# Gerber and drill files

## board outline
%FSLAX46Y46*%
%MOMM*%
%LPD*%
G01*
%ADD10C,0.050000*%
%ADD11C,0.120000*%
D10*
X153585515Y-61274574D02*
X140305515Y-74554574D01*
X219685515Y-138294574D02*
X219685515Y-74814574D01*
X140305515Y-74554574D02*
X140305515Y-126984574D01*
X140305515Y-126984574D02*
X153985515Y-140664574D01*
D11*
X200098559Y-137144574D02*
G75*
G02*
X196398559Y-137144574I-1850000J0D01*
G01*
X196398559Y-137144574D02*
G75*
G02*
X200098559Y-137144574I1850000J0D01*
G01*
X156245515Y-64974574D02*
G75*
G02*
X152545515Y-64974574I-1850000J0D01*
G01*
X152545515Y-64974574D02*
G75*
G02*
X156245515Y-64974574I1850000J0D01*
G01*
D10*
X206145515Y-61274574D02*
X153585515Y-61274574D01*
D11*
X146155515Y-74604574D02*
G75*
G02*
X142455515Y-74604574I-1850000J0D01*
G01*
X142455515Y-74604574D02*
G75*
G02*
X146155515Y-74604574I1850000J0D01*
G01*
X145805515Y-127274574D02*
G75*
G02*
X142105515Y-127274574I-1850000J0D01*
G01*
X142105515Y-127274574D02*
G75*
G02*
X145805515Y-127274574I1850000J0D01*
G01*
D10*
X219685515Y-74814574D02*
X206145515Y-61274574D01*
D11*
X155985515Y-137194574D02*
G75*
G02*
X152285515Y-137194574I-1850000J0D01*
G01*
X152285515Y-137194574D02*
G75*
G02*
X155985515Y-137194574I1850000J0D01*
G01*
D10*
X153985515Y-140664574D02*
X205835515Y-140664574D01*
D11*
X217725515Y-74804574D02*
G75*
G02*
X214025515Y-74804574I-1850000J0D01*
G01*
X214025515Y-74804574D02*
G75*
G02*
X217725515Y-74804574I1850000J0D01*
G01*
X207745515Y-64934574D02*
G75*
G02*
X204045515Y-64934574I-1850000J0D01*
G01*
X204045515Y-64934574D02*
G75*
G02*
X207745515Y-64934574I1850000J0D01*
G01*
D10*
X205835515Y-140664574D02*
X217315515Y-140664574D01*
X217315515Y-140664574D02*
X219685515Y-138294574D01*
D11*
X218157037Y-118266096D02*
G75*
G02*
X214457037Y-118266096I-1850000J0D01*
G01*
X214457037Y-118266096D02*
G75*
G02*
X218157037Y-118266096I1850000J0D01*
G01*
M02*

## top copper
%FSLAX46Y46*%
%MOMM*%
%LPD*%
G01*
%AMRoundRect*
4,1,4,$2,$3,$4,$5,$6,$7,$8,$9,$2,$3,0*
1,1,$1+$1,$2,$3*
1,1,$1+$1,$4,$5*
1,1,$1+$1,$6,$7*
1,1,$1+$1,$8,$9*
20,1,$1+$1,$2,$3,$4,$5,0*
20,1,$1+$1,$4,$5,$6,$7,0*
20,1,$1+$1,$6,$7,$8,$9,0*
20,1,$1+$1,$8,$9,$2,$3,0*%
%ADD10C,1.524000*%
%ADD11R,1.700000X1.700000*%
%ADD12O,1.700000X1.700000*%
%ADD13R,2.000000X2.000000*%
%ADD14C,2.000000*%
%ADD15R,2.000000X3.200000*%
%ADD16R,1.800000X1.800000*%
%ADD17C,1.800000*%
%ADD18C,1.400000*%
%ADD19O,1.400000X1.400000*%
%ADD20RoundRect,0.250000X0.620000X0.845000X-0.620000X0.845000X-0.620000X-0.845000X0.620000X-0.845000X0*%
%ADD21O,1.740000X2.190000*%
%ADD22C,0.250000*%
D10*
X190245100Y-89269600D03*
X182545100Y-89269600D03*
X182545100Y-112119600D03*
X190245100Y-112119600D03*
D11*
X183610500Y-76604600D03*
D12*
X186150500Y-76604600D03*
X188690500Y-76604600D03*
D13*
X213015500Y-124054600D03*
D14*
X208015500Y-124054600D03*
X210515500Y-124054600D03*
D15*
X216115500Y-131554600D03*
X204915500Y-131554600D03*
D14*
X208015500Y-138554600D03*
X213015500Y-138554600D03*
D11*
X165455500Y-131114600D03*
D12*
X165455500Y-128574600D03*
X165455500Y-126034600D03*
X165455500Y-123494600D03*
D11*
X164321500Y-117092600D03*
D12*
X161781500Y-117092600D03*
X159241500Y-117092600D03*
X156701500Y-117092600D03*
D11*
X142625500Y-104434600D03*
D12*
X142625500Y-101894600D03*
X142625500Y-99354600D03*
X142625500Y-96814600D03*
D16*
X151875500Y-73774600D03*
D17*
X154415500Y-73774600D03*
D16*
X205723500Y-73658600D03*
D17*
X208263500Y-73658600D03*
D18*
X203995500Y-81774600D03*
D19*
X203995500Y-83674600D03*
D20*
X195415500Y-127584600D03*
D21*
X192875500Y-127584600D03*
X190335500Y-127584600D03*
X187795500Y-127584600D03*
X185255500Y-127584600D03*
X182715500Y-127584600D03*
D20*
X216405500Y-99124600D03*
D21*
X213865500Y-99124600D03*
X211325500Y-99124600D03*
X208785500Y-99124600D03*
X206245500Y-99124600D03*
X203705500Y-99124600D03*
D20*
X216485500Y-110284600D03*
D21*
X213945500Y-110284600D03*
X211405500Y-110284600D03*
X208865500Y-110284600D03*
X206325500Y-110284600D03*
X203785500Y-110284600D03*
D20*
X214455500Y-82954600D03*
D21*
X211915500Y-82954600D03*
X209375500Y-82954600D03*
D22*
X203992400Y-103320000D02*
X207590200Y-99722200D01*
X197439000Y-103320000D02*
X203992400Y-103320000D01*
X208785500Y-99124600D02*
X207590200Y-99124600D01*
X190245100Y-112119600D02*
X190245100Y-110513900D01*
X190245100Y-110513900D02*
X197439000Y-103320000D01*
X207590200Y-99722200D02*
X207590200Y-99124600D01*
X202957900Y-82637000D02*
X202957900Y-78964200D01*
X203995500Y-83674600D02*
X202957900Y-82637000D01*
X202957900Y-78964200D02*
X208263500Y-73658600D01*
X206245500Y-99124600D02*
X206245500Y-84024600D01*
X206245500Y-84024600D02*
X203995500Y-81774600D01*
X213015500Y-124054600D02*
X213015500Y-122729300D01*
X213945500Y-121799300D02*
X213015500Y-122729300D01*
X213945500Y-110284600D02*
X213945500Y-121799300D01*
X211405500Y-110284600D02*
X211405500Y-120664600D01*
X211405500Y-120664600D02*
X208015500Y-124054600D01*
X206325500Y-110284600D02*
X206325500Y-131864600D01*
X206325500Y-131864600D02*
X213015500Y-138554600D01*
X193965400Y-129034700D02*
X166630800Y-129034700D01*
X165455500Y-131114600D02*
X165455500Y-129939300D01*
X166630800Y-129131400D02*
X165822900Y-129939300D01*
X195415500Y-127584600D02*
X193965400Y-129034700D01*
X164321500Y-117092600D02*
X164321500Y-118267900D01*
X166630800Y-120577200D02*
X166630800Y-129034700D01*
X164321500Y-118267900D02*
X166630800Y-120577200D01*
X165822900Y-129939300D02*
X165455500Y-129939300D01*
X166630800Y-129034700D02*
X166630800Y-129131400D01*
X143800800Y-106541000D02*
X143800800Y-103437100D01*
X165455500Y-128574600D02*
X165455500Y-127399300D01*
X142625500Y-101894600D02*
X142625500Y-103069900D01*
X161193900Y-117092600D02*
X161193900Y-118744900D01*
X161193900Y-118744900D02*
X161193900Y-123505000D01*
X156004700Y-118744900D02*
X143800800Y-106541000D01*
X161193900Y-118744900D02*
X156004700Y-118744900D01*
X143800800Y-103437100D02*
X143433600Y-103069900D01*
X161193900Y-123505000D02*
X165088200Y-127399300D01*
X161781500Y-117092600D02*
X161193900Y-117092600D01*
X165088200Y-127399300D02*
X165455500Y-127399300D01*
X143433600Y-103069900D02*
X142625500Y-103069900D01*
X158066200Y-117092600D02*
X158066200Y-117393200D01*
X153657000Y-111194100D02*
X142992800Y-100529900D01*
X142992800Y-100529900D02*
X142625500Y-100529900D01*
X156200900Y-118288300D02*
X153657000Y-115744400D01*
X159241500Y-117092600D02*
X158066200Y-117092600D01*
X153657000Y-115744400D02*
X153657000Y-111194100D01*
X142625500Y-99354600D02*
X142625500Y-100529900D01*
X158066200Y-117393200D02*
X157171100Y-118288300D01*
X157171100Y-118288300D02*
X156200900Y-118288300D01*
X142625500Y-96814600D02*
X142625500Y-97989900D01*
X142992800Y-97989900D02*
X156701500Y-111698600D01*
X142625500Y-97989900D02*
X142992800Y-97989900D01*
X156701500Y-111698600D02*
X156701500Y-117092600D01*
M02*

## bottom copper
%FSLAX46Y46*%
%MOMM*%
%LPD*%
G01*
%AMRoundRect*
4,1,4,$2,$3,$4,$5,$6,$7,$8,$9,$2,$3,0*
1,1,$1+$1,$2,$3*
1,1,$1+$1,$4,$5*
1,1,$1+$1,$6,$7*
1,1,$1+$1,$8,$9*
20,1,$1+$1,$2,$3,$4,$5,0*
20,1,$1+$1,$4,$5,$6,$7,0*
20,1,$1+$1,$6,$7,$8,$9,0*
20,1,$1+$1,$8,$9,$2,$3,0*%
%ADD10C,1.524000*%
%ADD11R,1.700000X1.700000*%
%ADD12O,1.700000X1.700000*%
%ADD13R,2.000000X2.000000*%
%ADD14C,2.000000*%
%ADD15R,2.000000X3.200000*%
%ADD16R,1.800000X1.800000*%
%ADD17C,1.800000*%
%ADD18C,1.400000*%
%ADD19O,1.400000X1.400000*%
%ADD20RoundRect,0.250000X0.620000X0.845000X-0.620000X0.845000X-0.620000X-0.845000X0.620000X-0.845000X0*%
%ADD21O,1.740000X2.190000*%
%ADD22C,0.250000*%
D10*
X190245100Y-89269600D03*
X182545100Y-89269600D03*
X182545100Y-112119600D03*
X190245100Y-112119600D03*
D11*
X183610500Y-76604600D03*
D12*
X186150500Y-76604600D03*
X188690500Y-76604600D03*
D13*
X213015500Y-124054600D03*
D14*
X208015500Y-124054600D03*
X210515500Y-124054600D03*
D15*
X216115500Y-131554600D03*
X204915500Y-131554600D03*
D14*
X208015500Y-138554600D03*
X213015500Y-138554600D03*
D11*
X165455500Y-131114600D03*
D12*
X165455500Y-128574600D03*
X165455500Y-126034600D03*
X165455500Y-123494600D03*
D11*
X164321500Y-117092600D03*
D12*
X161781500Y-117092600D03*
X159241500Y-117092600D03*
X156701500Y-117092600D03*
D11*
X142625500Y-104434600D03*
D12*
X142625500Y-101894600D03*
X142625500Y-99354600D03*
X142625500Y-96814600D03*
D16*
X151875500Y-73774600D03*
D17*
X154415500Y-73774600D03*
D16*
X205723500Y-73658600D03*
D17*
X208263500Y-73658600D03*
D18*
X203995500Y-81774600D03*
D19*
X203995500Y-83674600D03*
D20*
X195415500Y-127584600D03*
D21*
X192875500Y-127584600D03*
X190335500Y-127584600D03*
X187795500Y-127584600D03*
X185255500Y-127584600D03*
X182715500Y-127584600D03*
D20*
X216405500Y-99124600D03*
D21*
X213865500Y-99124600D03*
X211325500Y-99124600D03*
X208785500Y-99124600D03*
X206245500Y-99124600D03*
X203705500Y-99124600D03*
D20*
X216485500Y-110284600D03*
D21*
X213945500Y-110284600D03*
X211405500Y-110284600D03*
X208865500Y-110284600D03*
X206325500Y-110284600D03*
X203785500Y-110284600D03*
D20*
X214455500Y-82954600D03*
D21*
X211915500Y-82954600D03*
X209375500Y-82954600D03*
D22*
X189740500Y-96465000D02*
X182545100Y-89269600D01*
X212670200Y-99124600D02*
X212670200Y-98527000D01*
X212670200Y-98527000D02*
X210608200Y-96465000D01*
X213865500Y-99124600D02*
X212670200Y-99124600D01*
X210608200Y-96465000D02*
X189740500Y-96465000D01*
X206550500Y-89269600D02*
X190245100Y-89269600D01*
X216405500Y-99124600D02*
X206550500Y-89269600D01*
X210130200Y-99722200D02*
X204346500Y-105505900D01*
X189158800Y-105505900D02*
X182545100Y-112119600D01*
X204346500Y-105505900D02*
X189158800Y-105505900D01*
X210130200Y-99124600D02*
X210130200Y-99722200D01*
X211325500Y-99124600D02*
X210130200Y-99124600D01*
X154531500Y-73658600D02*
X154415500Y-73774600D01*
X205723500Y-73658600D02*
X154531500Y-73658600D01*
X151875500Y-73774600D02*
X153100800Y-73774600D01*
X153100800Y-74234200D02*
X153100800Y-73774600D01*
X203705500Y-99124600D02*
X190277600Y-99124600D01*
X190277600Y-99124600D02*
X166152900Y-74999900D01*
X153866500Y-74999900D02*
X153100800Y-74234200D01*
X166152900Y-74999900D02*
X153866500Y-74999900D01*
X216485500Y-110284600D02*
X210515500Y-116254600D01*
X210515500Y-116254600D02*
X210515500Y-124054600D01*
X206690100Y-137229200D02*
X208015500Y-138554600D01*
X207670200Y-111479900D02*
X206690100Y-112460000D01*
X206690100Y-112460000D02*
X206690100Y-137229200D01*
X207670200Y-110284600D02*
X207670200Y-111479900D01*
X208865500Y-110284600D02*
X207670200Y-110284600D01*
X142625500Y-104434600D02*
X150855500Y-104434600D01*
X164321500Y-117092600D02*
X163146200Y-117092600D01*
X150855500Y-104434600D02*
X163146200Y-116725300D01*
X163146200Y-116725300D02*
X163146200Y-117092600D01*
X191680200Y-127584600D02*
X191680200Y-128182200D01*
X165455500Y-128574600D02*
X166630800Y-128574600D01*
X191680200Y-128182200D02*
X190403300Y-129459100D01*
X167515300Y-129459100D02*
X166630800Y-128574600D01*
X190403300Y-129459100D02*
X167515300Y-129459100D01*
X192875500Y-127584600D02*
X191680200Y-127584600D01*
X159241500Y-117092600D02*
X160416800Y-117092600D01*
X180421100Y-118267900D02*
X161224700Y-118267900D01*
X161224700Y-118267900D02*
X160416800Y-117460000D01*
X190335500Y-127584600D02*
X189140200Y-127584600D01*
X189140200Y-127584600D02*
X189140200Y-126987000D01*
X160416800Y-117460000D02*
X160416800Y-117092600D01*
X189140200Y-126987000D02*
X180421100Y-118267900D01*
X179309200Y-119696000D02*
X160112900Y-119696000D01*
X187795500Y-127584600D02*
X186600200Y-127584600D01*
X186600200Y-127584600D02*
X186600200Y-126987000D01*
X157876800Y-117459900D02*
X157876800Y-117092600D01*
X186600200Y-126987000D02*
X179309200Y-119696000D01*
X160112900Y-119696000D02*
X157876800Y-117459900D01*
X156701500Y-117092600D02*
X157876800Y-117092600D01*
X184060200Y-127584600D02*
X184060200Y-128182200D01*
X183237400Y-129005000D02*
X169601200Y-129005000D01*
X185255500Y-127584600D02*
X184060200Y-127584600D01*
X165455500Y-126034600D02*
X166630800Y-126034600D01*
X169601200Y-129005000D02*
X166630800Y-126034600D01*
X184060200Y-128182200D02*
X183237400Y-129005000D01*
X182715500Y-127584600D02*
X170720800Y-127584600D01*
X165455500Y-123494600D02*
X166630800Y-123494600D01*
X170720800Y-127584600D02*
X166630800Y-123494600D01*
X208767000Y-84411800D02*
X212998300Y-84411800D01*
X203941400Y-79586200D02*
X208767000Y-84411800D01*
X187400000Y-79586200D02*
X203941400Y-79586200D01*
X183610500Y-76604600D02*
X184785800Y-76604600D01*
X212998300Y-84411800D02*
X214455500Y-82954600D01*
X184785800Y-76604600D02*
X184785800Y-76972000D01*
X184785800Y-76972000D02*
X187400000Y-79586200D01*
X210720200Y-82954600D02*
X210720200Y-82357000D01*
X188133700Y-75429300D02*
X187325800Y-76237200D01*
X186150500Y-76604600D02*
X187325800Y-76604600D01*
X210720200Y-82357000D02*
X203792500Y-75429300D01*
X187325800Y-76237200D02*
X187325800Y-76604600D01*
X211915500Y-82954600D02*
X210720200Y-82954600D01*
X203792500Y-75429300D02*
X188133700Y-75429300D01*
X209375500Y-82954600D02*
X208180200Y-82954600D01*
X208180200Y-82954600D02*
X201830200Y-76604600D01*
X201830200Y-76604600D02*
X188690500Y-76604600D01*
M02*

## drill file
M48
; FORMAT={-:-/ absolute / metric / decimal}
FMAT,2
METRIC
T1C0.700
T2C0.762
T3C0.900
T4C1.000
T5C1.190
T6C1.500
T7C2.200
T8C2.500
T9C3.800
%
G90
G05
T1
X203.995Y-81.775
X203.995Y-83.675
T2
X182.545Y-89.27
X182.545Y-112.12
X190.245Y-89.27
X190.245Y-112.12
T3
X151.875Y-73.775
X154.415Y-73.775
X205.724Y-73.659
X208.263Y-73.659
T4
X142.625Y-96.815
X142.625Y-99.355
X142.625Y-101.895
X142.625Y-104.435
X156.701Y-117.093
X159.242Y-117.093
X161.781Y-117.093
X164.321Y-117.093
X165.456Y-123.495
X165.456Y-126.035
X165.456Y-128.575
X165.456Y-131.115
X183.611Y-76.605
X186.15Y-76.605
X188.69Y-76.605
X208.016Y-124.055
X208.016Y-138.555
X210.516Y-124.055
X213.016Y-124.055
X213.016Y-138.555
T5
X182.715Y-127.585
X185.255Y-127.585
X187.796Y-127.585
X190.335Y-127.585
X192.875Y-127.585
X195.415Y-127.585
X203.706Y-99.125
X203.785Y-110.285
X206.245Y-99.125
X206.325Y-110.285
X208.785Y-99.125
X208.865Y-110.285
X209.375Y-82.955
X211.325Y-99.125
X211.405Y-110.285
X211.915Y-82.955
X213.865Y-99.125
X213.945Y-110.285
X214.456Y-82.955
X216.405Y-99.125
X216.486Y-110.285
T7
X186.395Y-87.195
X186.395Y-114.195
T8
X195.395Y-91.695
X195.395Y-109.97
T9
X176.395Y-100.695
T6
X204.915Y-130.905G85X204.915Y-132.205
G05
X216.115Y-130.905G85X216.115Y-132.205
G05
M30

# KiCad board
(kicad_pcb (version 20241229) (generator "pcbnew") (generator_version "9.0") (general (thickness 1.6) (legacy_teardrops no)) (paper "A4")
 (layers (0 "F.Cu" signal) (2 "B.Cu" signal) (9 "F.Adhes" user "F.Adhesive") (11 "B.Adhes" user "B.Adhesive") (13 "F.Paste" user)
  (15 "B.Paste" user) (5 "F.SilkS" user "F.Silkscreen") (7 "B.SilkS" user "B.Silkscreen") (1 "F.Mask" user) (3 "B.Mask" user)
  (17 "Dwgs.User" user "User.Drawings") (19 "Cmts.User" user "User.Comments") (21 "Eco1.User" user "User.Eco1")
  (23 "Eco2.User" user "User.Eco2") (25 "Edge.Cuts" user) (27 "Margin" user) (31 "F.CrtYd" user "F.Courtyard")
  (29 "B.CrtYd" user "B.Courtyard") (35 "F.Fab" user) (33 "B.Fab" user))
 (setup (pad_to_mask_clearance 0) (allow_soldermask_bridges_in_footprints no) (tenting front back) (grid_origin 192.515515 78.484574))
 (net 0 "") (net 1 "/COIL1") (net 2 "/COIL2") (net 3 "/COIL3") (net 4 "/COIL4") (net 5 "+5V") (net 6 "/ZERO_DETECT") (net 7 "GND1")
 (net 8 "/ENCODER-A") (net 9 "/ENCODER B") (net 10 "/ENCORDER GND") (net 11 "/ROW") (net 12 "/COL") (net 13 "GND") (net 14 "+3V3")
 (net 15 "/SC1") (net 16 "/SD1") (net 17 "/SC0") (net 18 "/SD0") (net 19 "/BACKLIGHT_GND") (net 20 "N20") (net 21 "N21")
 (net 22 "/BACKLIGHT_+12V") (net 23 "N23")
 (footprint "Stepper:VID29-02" (layer "F.Cu") (at 186.3951 100.8596 -90)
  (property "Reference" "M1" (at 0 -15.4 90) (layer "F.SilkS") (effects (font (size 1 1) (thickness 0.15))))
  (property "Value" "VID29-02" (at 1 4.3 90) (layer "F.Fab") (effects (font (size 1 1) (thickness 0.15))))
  (pad "" np_thru_hole circle (at -13.665 0 270) (size 2.2 2.2) (drill 2.2) (layers "*.Cu" "*.Mask"))
  (pad "" np_thru_hole circle (at -9.165 -9 270) (size 2.5 2.5) (drill 2.5) (layers "*.Cu" "*.Mask"))
  (pad "" np_thru_hole circle (at -0.165 10 270) (size 3.8 3.8) (drill 3.8) (layers "*.Cu" "*.Mask"))
  (pad "" np_thru_hole circle (at 9.11 -9 270) (size 2.5 2.5) (drill 2.5) (layers "*.Cu" "*.Mask"))
  (pad "" np_thru_hole circle (at 13.335 0 270) (size 2.2 2.2) (drill 2.2) (layers "*.Cu" "*.Mask"))
  (pad "1" thru_hole circle (at -11.59 -3.85 270) (size 1.524 1.524) (drill 0.762) (layers "*.Cu" "*.Mask") (remove_unused_layers no)
   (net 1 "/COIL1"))
  (pad "2" thru_hole circle (at -11.59 3.85 270) (size 1.524 1.524) (drill 0.762) (layers "*.Cu" "*.Mask") (remove_unused_layers no)
   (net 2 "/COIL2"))
  (pad "3" thru_hole circle (at 11.26 3.85 270) (size 1.524 1.524) (drill 0.762) (layers "*.Cu" "*.Mask") (remove_unused_layers no)
   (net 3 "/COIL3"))
  (pad "4" thru_hole circle (at 11.26 -3.85 270) (size 1.524 1.524) (drill 0.762) (layers "*.Cu" "*.Mask") (remove_unused_layers no)
   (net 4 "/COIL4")))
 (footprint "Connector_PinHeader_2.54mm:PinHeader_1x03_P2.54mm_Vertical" (layer "F.Cu") (at 183.6105 76.6046 90)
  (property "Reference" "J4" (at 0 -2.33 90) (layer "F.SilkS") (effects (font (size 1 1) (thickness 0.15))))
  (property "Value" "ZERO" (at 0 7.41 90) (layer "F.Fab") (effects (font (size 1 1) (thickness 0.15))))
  (pad "1" thru_hole rect (at 0 0 90) (size 1.7 1.7) (drill 1) (layers "*.Cu" "*.Mask") (remove_unused_layers no) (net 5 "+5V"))
  (pad "2" thru_hole oval (at 0 2.54 90) (size 1.7 1.7) (drill 1) (layers "*.Cu" "*.Mask") (remove_unused_layers no) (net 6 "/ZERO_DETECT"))
  (pad "3" thru_hole oval (at 0 5.08 90) (size 1.7 1.7) (drill 1) (layers "*.Cu" "*.Mask") (remove_unused_layers no) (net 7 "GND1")))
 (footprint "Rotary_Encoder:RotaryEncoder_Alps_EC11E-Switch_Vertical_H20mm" (layer "F.Cu") (at 213.0155 124.0546 -90)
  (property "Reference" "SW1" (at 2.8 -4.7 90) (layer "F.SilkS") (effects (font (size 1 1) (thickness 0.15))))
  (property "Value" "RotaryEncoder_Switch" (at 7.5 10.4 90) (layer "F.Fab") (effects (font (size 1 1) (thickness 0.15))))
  (pad "A" thru_hole rect (at 0 0 270) (size 2 2) (drill 1) (layers "*.Cu" "*.Mask") (remove_unused_layers no) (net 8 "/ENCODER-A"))
  (pad "B" thru_hole circle (at 0 5 270) (size 2 2) (drill 1) (layers "*.Cu" "*.Mask") (remove_unused_layers no) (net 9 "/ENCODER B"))
  (pad "C" thru_hole circle (at 0 2.5 270) (size 2 2) (drill 1) (layers "*.Cu" "*.Mask") (remove_unused_layers no) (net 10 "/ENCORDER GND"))
  (pad "MP" thru_hole rect (at 7.5 -3.1 270) (size 3.2 2) (drill oval 2.8 1.5) (layers "*.Cu" "*.Mask") (remove_unused_layers no))
  (pad "MP" thru_hole rect (at 7.5 8.1 270) (size 3.2 2) (drill oval 2.8 1.5) (layers "*.Cu" "*.Mask") (remove_unused_layers no))
  (pad "S1" thru_hole circle (at 14.5 5 270) (size 2 2) (drill 1) (layers "*.Cu" "*.Mask") (remove_unused_layers no) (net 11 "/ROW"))
  (pad "S2" thru_hole circle (at 14.5 0 270) (size 2 2) (drill 1) (layers "*.Cu" "*.Mask") (remove_unused_layers no) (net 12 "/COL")))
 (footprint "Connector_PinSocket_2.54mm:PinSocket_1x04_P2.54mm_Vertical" (layer "F.Cu") (at 165.4555 131.1146 180)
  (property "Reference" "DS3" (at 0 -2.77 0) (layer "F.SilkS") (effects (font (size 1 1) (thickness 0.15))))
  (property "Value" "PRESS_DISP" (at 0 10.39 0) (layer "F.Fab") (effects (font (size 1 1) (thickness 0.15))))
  (pad "1" thru_hole rect (at 0 0 180) (size 1.7 1.7) (drill 1) (layers "*.Cu" "*.Mask") (remove_unused_layers no) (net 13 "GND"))
  (pad "2" thru_hole oval (at 0 2.54 180) (size 1.7 1.7) (drill 1) (layers "*.Cu" "*.Mask") (remove_unused_layers no) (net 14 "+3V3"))
  (pad "3" thru_hole oval (at 0 5.08 180) (size 1.7 1.7) (drill 1) (layers "*.Cu" "*.Mask") (remove_unused_layers no) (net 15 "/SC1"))
  (pad "4" thru_hole oval (at 0 7.62 180) (size 1.7 1.7) (drill 1) (layers "*.Cu" "*.Mask") (remove_unused_layers no) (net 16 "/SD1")))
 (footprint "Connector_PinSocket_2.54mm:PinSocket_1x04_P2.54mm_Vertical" (layer "F.Cu") (at 164.3215 117.0926 -90)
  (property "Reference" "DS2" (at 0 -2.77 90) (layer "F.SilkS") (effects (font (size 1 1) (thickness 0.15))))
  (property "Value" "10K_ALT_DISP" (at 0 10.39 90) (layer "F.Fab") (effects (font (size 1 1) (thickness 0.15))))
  (pad "1" thru_hole rect (at 0 0 270) (size 1.7 1.7) (drill 1) (layers "*.Cu" "*.Mask") (remove_unused_layers no) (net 13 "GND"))
  (pad "2" thru_hole oval (at 0 2.54 270) (size 1.7 1.7) (drill 1) (layers "*.Cu" "*.Mask") (remove_unused_layers no) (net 14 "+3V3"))
  (pad "3" thru_hole oval (at 0 5.08 270) (size 1.7 1.7) (drill 1) (layers "*.Cu" "*.Mask") (remove_unused_layers no) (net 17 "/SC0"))
  (pad "4" thru_hole oval (at 0 7.62 270) (size 1.7 1.7) (drill 1) (layers "*.Cu" "*.Mask") (remove_unused_layers no) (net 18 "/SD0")))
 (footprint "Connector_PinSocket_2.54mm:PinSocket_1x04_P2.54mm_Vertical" (layer "F.Cu") (at 142.6255 104.4346 180)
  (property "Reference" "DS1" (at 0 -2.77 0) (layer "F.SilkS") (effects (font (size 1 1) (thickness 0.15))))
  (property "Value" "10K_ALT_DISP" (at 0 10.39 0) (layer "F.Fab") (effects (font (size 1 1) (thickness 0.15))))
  (pad "1" thru_hole rect (at 0 0 180) (size 1.7 1.7) (drill 1) (layers "*.Cu" "*.Mask") (remove_unused_layers no) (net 13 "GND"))
  (pad "2" thru_hole oval (at 0 2.54 180) (size 1.7 1.7) (drill 1) (layers "*.Cu" "*.Mask") (remove_unused_layers no) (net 14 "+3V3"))
  (pad "3" thru_hole oval (at 0 5.08 180) (size 1.7 1.7) (drill 1) (layers "*.Cu" "*.Mask") (remove_unused_layers no) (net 17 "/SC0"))
  (pad "4" thru_hole oval (at 0 7.62 180) (size 1.7 1.7) (drill 1) (layers "*.Cu" "*.Mask") (remove_unused_layers no) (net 18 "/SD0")))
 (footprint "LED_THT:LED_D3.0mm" (layer "F.Cu") (at 151.8755 73.7746)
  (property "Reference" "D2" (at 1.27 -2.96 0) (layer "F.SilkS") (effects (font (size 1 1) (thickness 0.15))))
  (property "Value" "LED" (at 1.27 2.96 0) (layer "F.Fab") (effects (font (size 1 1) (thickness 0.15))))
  (pad "1" thru_hole rect (at 0 0) (size 1.8 1.8) (drill 0.9) (layers "*.Cu" "*.Mask") (remove_unused_layers no) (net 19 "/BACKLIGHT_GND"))
  (pad "2" thru_hole circle (at 2.54 0) (size 1.8 1.8) (drill 0.9) (layers "*.Cu" "*.Mask") (remove_unused_layers no) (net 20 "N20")))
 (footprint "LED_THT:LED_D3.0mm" (layer "F.Cu") (at 205.7235 73.6586)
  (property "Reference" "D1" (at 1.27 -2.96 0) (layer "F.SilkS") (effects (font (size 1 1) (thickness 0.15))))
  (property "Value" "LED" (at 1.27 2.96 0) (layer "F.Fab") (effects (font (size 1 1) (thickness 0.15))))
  (pad "1" thru_hole rect (at 0 0) (size 1.8 1.8) (drill 0.9) (layers "*.Cu" "*.Mask") (remove_unused_layers no) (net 20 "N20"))
  (pad "2" thru_hole circle (at 2.54 0) (size 1.8 1.8) (drill 0.9) (layers "*.Cu" "*.Mask") (remove_unused_layers no) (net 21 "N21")))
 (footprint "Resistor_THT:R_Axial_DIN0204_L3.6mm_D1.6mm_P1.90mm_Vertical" (layer "B.Cu") (at 203.9955 81.7746 -90)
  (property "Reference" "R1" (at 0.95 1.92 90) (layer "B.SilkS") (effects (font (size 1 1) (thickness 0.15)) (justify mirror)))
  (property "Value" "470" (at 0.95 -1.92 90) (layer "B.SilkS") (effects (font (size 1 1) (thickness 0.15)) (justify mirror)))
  (pad "1" thru_hole circle (at 0 0 270) (size 1.4 1.4) (drill 0.7) (layers "*.Cu" "*.Mask") (remove_unused_layers no)
   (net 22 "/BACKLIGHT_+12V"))
  (pad "2" thru_hole oval (at 1.9 0 270) (size 1.4 1.4) (drill 0.7) (layers "*.Cu" "*.Mask") (remove_unused_layers no) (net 21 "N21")))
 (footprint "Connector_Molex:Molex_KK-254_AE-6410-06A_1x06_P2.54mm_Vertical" (layer "B.Cu") (at 195.4155 127.5846 180)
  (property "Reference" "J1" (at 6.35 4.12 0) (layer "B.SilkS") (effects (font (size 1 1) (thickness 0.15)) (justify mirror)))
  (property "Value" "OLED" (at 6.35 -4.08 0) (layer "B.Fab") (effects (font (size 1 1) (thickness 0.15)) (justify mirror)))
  (pad "1" thru_hole roundrect (at 0 0 180) (size 1.74 2.19) (drill 1.19) (layers "*.Cu" "*.Mask") (remove_unused_layers no)
   (roundrect_rratio 0.1436781609) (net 13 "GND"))
  (pad "2" thru_hole oval (at 2.54 0 180) (size 1.74 2.19) (drill 1.19) (layers "*.Cu" "*.Mask") (remove_unused_layers no) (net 14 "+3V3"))
  (pad "3" thru_hole oval (at 5.08 0 180) (size 1.74 2.19) (drill 1.19) (layers "*.Cu" "*.Mask") (remove_unused_layers no) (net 17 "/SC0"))
  (pad "4" thru_hole oval (at 7.62 0 180) (size 1.74 2.19) (drill 1.19) (layers "*.Cu" "*.Mask") (remove_unused_layers no) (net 18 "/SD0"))
  (pad "5" thru_hole oval (at 10.16 0 180) (size 1.74 2.19) (drill 1.19) (layers "*.Cu" "*.Mask") (remove_unused_layers no) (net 15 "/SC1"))
  (pad "6" thru_hole oval (at 12.7 0 180) (size 1.74 2.19) (drill 1.19) (layers "*.Cu" "*.Mask") (remove_unused_layers no) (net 16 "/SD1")))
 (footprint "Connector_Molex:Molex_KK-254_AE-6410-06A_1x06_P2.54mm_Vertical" (layer "B.Cu") (at 216.4055 99.1246 180)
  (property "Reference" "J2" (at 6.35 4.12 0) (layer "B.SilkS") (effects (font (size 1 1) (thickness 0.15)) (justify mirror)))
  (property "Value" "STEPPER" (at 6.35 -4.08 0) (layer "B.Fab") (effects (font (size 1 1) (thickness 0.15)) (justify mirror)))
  (pad "1" thru_hole roundrect (at 0 0 180) (size 1.74 2.19) (drill 1.19) (layers "*.Cu" "*.Mask") (remove_unused_layers no)
   (roundrect_rratio 0.1436781609) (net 1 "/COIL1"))
  (pad "2" thru_hole oval (at 2.54 0 180) (size 1.74 2.19) (drill 1.19) (layers "*.Cu" "*.Mask") (remove_unused_layers no) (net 2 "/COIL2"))
  (pad "3" thru_hole oval (at 5.08 0 180) (size 1.74 2.19) (drill 1.19) (layers "*.Cu" "*.Mask") (remove_unused_layers no) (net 3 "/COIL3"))
  (pad "4" thru_hole oval (at 7.62 0 180) (size 1.74 2.19) (drill 1.19) (layers "*.Cu" "*.Mask") (remove_unused_layers no) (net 4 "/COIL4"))
  (pad "5" thru_hole oval (at 10.16 0 180) (size 1.74 2.19) (drill 1.19) (layers "*.Cu" "*.Mask") (remove_unused_layers no)
   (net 22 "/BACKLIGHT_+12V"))
  (pad "6" thru_hole oval (at 12.7 0 180) (size 1.74 2.19) (drill 1.19) (layers "*.Cu" "*.Mask") (remove_unused_layers no)
   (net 19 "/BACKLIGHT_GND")))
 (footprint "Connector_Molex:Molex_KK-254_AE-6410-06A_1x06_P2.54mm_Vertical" (layer "B.Cu") (at 216.4855 110.2846 180)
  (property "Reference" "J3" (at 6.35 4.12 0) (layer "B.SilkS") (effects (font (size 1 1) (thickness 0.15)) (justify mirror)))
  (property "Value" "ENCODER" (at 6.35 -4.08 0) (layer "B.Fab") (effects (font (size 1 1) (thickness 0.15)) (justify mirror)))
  (pad "1" thru_hole roundrect (at 0 0 180) (size 1.74 2.19) (drill 1.19) (layers "*.Cu" "*.Mask") (remove_unused_layers no)
   (roundrect_rratio 0.1436781609) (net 10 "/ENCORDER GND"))
  (pad "2" thru_hole oval (at 2.54 0 180) (size 1.74 2.19) (drill 1.19) (layers "*.Cu" "*.Mask") (remove_unused_layers no)
   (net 8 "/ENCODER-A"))
  (pad "3" thru_hole oval (at 5.08 0 180) (size 1.74 2.19) (drill 1.19) (layers "*.Cu" "*.Mask") (remove_unused_layers no)
   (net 9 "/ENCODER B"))
  (pad "4" thru_hole oval (at 7.62 0 180) (size 1.74 2.19) (drill 1.19) (layers "*.Cu" "*.Mask") (remove_unused_layers no) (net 11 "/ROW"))
  (pad "5" thru_hole oval (at 10.16 0 180) (size 1.74 2.19) (drill 1.19) (layers "*.Cu" "*.Mask") (remove_unused_layers no) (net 12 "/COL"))
  (pad "6" thru_hole oval (at 12.7 0 180) (size 1.74 2.19) (drill 1.19) (layers "*.Cu" "*.Mask") (remove_unused_layers no) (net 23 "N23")))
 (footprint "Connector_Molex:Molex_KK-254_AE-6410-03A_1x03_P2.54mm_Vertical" (layer "B.Cu") (at 214.4555 82.9546 180)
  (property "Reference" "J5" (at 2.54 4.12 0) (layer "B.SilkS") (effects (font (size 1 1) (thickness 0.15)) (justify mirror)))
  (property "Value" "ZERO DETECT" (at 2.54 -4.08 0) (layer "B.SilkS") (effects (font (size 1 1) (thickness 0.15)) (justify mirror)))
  (pad "1" thru_hole roundrect (at 0 0 180) (size 1.74 2.19) (drill 1.19) (layers "*.Cu" "*.Mask") (remove_unused_layers no)
   (roundrect_rratio 0.1436781609) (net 5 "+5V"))
  (pad "2" thru_hole oval (at 2.54 0 180) (size 1.74 2.19) (drill 1.19) (layers "*.Cu" "*.Mask") (remove_unused_layers no)
   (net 6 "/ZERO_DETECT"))
  (pad "3" thru_hole oval (at 5.08 0 180) (size 1.74 2.19) (drill 1.19) (layers "*.Cu" "*.Mask") (remove_unused_layers no) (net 7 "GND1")))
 (gr_line (start 153.585515 61.274574) (end 140.305515 74.554574) (stroke (width 0.05) (type solid)) (layer "Edge.Cuts"))
 (gr_line (start 219.685515 138.294574) (end 219.685515 74.814574) (stroke (width 0.05) (type solid)) (layer "Edge.Cuts"))
 (gr_line (start 140.305515 74.554574) (end 140.305515 126.984574) (stroke (width 0.05) (type solid)) (layer "Edge.Cuts"))
 (gr_line (start 140.305515 126.984574) (end 153.985515 140.664574) (stroke (width 0.05) (type solid)) (layer "Edge.Cuts"))
 (gr_circle (center 198.248559 137.144574) (end 200.098559 137.144574) (stroke (width 0.12) (type solid)) (fill no) (layer "Edge.Cuts"))
 (gr_circle (center 154.395515 64.974574) (end 156.245515 64.974574) (stroke (width 0.12) (type solid)) (fill no) (layer "Edge.Cuts"))
 (gr_line (start 206.145515 61.274574) (end 153.585515 61.274574) (stroke (width 0.05) (type solid)) (layer "Edge.Cuts"))
 (gr_circle (center 144.305515 74.604574) (end 146.155515 74.604574) (stroke (width 0.12) (type solid)) (fill no) (layer "Edge.Cuts"))
 (gr_circle (center 143.955515 127.274574) (end 145.805515 127.274574) (stroke (width 0.12) (type solid)) (fill no) (layer "Edge.Cuts"))
 (gr_line (start 219.685515 74.814574) (end 206.145515 61.274574) (stroke (width 0.05) (type solid)) (layer "Edge.Cuts"))
 (gr_circle (center 154.135515 137.194574) (end 155.985515 137.194574) (stroke (width 0.12) (type solid)) (fill no) (layer "Edge.Cuts"))
 (gr_line (start 153.985515 140.664574) (end 205.835515 140.664574) (stroke (width 0.05) (type solid)) (layer "Edge.Cuts"))
 (gr_circle (center 215.875515 74.804574) (end 217.725515 74.804574) (stroke (width 0.12) (type solid)) (fill no) (layer "Edge.Cuts"))
 (gr_circle (center 205.895515 64.934574) (end 207.745515 64.934574) (stroke (width 0.12) (type solid)) (fill no) (layer "Edge.Cuts"))
 (gr_line (start 205.835515 140.664574) (end 217.315515 140.664574) (stroke (width 0.05) (type solid)) (layer "Edge.Cuts"))
 (gr_line (start 217.315515 140.664574) (end 219.685515 138.294574) (stroke (width 0.05) (type solid)) (layer "Edge.Cuts"))
 (gr_circle (center 216.307037 118.266096) (end 218.157037 118.266096) (stroke (width 0.12) (type solid)) (fill no) (layer "Edge.Cuts"))
 (segment (start 189.7405 96.465) (end 182.5451 89.2696) (width 0.25) (layer "B.Cu") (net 2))
 (segment (start 212.6702 99.1246) (end 212.6702 98.527) (width 0.25) (layer "B.Cu") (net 2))
 (segment (start 212.6702 98.527) (end 210.6082 96.465) (width 0.25) (layer "B.Cu") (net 2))
 (segment (start 213.8655 99.1246) (end 212.6702 99.1246) (width 0.25) (layer "B.Cu") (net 2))
 (segment (start 210.6082 96.465) (end 189.7405 96.465) (width 0.25) (layer "B.Cu") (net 2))
 (segment (start 206.5505 89.2696) (end 190.2451 89.2696) (width 0.25) (layer "B.Cu") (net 1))
 (segment (start 216.4055 99.1246) (end 206.5505 89.2696) (width 0.25) (layer "B.Cu") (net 1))
 (segment (start 203.9924 103.32) (end 207.5902 99.7222) (width 0.25) (layer "F.Cu") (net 4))
 (segment (start 197.439 103.32) (end 203.9924 103.32) (width 0.25) (layer "F.Cu") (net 4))
 (segment (start 208.7855 99.1246) (end 207.5902 99.1246) (width 0.25) (layer "F.Cu") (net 4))
 (segment (start 190.2451 112.1196) (end 190.2451 110.5139) (width 0.25) (layer "F.Cu") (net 4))
 (segment (start 190.2451 110.5139) (end 197.439 103.32) (width 0.25) (layer "F.Cu") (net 4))
 (segment (start 207.5902 99.7222) (end 207.5902 99.1246) (width 0.25) (layer "F.Cu") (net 4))
 (segment (start 210.1302 99.7222) (end 204.3465 105.5059) (width 0.25) (layer "B.Cu") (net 3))
 (segment (start 189.1588 105.5059) (end 182.5451 112.1196) (width 0.25) (layer "B.Cu") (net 3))
 (segment (start 204.3465 105.5059) (end 189.1588 105.5059) (width 0.25) (layer "B.Cu") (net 3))
 (segment (start 210.1302 99.1246) (end 210.1302 99.7222) (width 0.25) (layer "B.Cu") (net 3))
 (segment (start 211.3255 99.1246) (end 210.1302 99.1246) (width 0.25) (layer "B.Cu") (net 3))
 (segment (start 154.5315 73.6586) (end 154.4155 73.7746) (width 0.25) (layer "B.Cu") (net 20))
 (segment (start 205.7235 73.6586) (end 154.5315 73.6586) (width 0.25) (layer "B.Cu") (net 20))
 (segment (start 202.9579 82.637) (end 202.9579 78.9642) (width 0.25) (layer "F.Cu") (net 21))
 (segment (start 203.9955 83.6746) (end 202.9579 82.637) (width 0.25) (layer "F.Cu") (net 21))
 (segment (start 202.9579 78.9642) (end 208.2635 73.6586) (width 0.25) (layer "F.Cu") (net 21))
 (segment (start 151.8755 73.7746) (end 153.1008 73.7746) (width 0.25) (layer "B.Cu") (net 19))
 (segment (start 153.1008 74.2342) (end 153.1008 73.7746) (width 0.25) (layer "B.Cu") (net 19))
 (segment (start 203.7055 99.1246) (end 190.2776 99.1246) (width 0.25) (layer "B.Cu") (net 19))
 (segment (start 190.2776 99.1246) (end 166.1529 74.9999) (width 0.25) (layer "B.Cu") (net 19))
 (segment (start 153.8665 74.9999) (end 153.1008 74.2342) (width 0.25) (layer "B.Cu") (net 19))
 (segment (start 166.1529 74.9999) (end 153.8665 74.9999) (width 0.25) (layer "B.Cu") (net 19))
 (segment (start 206.2455 99.1246) (end 206.2455 84.0246) (width 0.25) (layer "F.Cu") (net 22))
 (segment (start 206.2455 84.0246) (end 203.9955 81.7746) (width 0.25) (layer "F.Cu") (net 22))
 (segment (start 216.4855 110.2846) (end 210.5155 116.2546) (width 0.25) (layer "B.Cu") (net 10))
 (segment (start 210.5155 116.2546) (end 210.5155 124.0546) (width 0.25) (layer "B.Cu") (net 10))
 (segment (start 213.0155 124.0546) (end 213.0155 122.7293) (width 0.25) (layer "F.Cu") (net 8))
 (segment (start 213.9455 121.7993) (end 213.0155 122.7293) (width 0.25) (layer "F.Cu") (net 8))
 (segment (start 213.9455 110.2846) (end 213.9455 121.7993) (width 0.25) (layer "F.Cu") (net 8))
 (segment (start 211.4055 110.2846) (end 211.4055 120.6646) (width 0.25) (layer "F.Cu") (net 9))
 (segment (start 211.4055 120.6646) (end 208.0155 124.0546) (width 0.25) (layer "F.Cu") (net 9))
 (segment (start 206.6901 137.2292) (end 208.0155 138.5546) (width 0.25) (layer "B.Cu") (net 11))
 (segment (start 207.6702 111.4799) (end 206.6901 112.46) (width 0.25) (layer "B.Cu") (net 11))
 (segment (start 206.6901 112.46) (end 206.6901 137.2292) (width 0.25) (layer "B.Cu") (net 11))
 (segment (start 207.6702 110.2846) (end 207.6702 111.4799) (width 0.25) (layer "B.Cu") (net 11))
 (segment (start 208.8655 110.2846) (end 207.6702 110.2846) (width 0.25) (layer "B.Cu") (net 11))
 (segment (start 206.3255 110.2846) (end 206.3255 131.8646) (width 0.25) (layer "F.Cu") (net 12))
 (segment (start 206.3255 131.8646) (end 213.0155 138.5546) (width 0.25) (layer "F.Cu") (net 12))
 (segment (start 193.9654 129.0347) (end 166.6308 129.0347) (width 0.25) (layer "F.Cu") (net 13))
 (segment (start 165.4555 131.1146) (end 165.4555 129.9393) (width 0.25) (layer "F.Cu") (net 13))
 (segment (start 166.6308 129.1314) (end 165.8229 129.9393) (width 0.25) (layer "F.Cu") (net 13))
 (segment (start 195.4155 127.5846) (end 193.9654 129.0347) (width 0.25) (layer "F.Cu") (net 13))
 (segment (start 164.3215 117.0926) (end 164.3215 118.2679) (width 0.25) (layer "F.Cu") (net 13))
 (segment (start 166.6308 120.5772) (end 166.6308 129.0347) (width 0.25) (layer "F.Cu") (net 13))
 (segment (start 164.3215 118.2679) (end 166.6308 120.5772) (width 0.25) (layer "F.Cu") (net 13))
 (segment (start 165.8229 129.9393) (end 165.4555 129.9393) (width 0.25) (layer "F.Cu") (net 13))
 (segment (start 166.6308 129.0347) (end 166.6308 129.1314) (width 0.25) (layer "F.Cu") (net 13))
 (segment (start 142.6255 104.4346) (end 150.8555 104.4346) (width 0.25) (layer "B.Cu") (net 13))
 (segment (start 164.3215 117.0926) (end 163.1462 117.0926) (width 0.25) (layer "B.Cu") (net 13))
 (segment (start 150.8555 104.4346) (end 163.1462 116.7253) (width 0.25) (layer "B.Cu") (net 13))
 (segment (start 163.1462 116.7253) (end 163.1462 117.0926) (width 0.25) (layer "B.Cu") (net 13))
 (segment (start 143.8008 106.541) (end 143.8008 103.4371) (width 0.25) (layer "F.Cu") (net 14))
 (segment (start 165.4555 128.5746) (end 165.4555 127.3993) (width 0.25) (layer "F.Cu") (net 14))
 (segment (start 142.6255 101.8946) (end 142.6255 103.0699) (width 0.25) (layer "F.Cu") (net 14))
 (segment (start 161.1939 117.0926) (end 161.1939 118.7449) (width 0.25) (layer "F.Cu") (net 14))
 (segment (start 161.1939 118.7449) (end 161.1939 123.505) (width 0.25) (layer "F.Cu") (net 14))
 (segment (start 156.0047 118.7449) (end 143.8008 106.541) (width 0.25) (layer "F.Cu") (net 14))
 (segment (start 161.1939 118.7449) (end 156.0047 118.7449) (width 0.25) (layer "F.Cu") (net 14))
 (segment (start 143.8008 103.4371) (end 143.4336 103.0699) (width 0.25) (layer "F.Cu") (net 14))
 (segment (start 161.1939 123.505) (end 165.0882 127.3993) (width 0.25) (layer "F.Cu") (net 14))
 (segment (start 161.7815 117.0926) (end 161.1939 117.0926) (width 0.25) (layer "F.Cu") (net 14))
 (segment (start 165.0882 127.3993) (end 165.4555 127.3993) (width 0.25) (layer "F.Cu") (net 14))
 (segment (start 143.4336 103.0699) (end 142.6255 103.0699) (width 0.25) (layer "F.Cu") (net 14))
 (segment (start 191.6802 127.5846) (end 191.6802 128.1822) (width 0.25) (layer "B.Cu") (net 14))
 (segment (start 165.4555 128.5746) (end 166.6308 128.5746) (width 0.25) (layer "B.Cu") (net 14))
 (segment (start 191.6802 128.1822) (end 190.4033 129.4591) (width 0.25) (layer "B.Cu") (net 14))
 (segment (start 167.5153 129.4591) (end 166.6308 128.5746) (width 0.25) (layer "B.Cu") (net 14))
 (segment (start 190.4033 129.4591) (end 167.5153 129.4591) (width 0.25) (layer "B.Cu") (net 14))
 (segment (start 192.8755 127.5846) (end 191.6802 127.5846) (width 0.25) (layer "B.Cu") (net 14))
 (segment (start 158.0662 117.0926) (end 158.0662 117.3932) (width 0.25) (layer "F.Cu") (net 17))
 (segment (start 153.657 111.1941) (end 142.9928 100.5299) (width 0.25) (layer "F.Cu") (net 17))
 (segment (start 142.9928 100.5299) (end 142.6255 100.5299) (width 0.25) (layer "F.Cu") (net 17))
 (segment (start 156.2009 118.2883) (end 153.657 115.7444) (width 0.25) (layer "F.Cu") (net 17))
 (segment (start 159.2415 117.0926) (end 158.0662 117.0926) (width 0.25) (layer "F.Cu") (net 17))
 (segment (start 153.657 115.7444) (end 153.657 111.1941) (width 0.25) (layer "F.Cu") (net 17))
 (segment (start 142.6255 99.3546) (end 142.6255 100.5299) (width 0.25) (layer "F.Cu") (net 17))
 (segment (start 158.0662 117.3932) (end 157.1711 118.2883) (width 0.25) (layer "F.Cu") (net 17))
 (segment (start 157.1711 118.2883) (end 156.2009 118.2883) (width 0.25) (layer "F.Cu") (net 17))
 (segment (start 159.2415 117.0926) (end 160.4168 117.0926) (width 0.25) (layer "B.Cu") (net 17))
 (segment (start 180.4211 118.2679) (end 161.2247 118.2679) (width 0.25) (layer "B.Cu") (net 17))
 (segment (start 161.2247 118.2679) (end 160.4168 117.46) (width 0.25) (layer "B.Cu") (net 17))
 (segment (start 190.3355 127.5846) (end 189.1402 127.5846) (width 0.25) (layer "B.Cu") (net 17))
 (segment (start 189.1402 127.5846) (end 189.1402 126.987) (width 0.25) (layer "B.Cu") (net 17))
 (segment (start 160.4168 117.46) (end 160.4168 117.0926) (width 0.25) (layer "B.Cu") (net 17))
 (segment (start 189.1402 126.987) (end 180.4211 118.2679) (width 0.25) (layer "B.Cu") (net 17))
 (segment (start 142.6255 96.8146) (end 142.6255 97.9899) (width 0.25) (layer "F.Cu") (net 18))
 (segment (start 142.9928 97.9899) (end 156.7015 111.6986) (width 0.25) (layer "F.Cu") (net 18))
 (segment (start 142.6255 97.9899) (end 142.9928 97.9899) (width 0.25) (layer "F.Cu") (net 18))
 (segment (start 156.7015 111.6986) (end 156.7015 117.0926) (width 0.25) (layer "F.Cu") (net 18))
 (segment (start 179.3092 119.696) (end 160.1129 119.696) (width 0.25) (layer "B.Cu") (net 18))
 (segment (start 187.7955 127.5846) (end 186.6002 127.5846) (width 0.25) (layer "B.Cu") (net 18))
 (segment (start 186.6002 127.5846) (end 186.6002 126.987) (width 0.25) (layer "B.Cu") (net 18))
 (segment (start 157.8768 117.4599) (end 157.8768 117.0926) (width 0.25) (layer "B.Cu") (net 18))
 (segment (start 186.6002 126.987) (end 179.3092 119.696) (width 0.25) (layer "B.Cu") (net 18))
 (segment (start 160.1129 119.696) (end 157.8768 117.4599) (width 0.25) (layer "B.Cu") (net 18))
 (segment (start 156.7015 117.0926) (end 157.8768 117.0926) (width 0.25) (layer "B.Cu") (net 18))
 (segment (start 184.0602 127.5846) (end 184.0602 128.1822) (width 0.25) (layer "B.Cu") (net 15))
 (segment (start 183.2374 129.005) (end 169.6012 129.005) (width 0.25) (layer "B.Cu") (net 15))
 (segment (start 185.2555 127.5846) (end 184.0602 127.5846) (width 0.25) (layer "B.Cu") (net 15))
 (segment (start 165.4555 126.0346) (end 166.6308 126.0346) (width 0.25) (layer "B.Cu") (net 15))
 (segment (start 169.6012 129.005) (end 166.6308 126.0346) (width 0.25) (layer "B.Cu") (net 15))
 (segment (start 184.0602 128.1822) (end 183.2374 129.005) (width 0.25) (layer "B.Cu") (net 15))
 (segment (start 182.7155 127.5846) (end 170.7208 127.5846) (width 0.25) (layer "B.Cu") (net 16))
 (segment (start 165.4555 123.4946) (end 166.6308 123.4946) (width 0.25) (layer "B.Cu") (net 16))
 (segment (start 170.7208 127.5846) (end 166.6308 123.4946) (width 0.25) (layer "B.Cu") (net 16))
 (segment (start 208.767 84.4118) (end 212.9983 84.4118) (width 0.25) (layer "B.Cu") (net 5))
 (segment (start 203.9414 79.5862) (end 208.767 84.4118) (width 0.25) (layer "B.Cu") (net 5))
 (segment (start 187.4 79.5862) (end 203.9414 79.5862) (width 0.25) (layer "B.Cu") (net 5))
 (segment (start 183.6105 76.6046) (end 184.7858 76.6046) (width 0.25) (layer "B.Cu") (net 5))
 (segment (start 212.9983 84.4118) (end 214.4555 82.9546) (width 0.25) (layer "B.Cu") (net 5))
 (segment (start 184.7858 76.6046) (end 184.7858 76.972) (width 0.25) (layer "B.Cu") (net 5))
 (segment (start 184.7858 76.972) (end 187.4 79.5862) (width 0.25) (layer "B.Cu") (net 5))
 (segment (start 210.7202 82.9546) (end 210.7202 82.357) (width 0.25) (layer "B.Cu") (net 6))
 (segment (start 188.1337 75.4293) (end 187.3258 76.2372) (width 0.25) (layer "B.Cu") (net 6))
 (segment (start 186.1505 76.6046) (end 187.3258 76.6046) (width 0.25) (layer "B.Cu") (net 6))
 (segment (start 210.7202 82.357) (end 203.7925 75.4293) (width 0.25) (layer "B.Cu") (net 6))
 (segment (start 187.3258 76.2372) (end 187.3258 76.6046) (width 0.25) (layer "B.Cu") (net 6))
 (segment (start 211.9155 82.9546) (end 210.7202 82.9546) (width 0.25) (layer "B.Cu") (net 6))
 (segment (start 203.7925 75.4293) (end 188.1337 75.4293) (width 0.25) (layer "B.Cu") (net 6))
 (segment (start 209.3755 82.9546) (end 208.1802 82.9546) (width 0.25) (layer "B.Cu") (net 7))
 (segment (start 208.1802 82.9546) (end 201.8302 76.6046) (width 0.25) (layer "B.Cu") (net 7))
 (segment (start 201.8302 76.6046) (end 188.6905 76.6046) (width 0.25) (layer "B.Cu") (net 7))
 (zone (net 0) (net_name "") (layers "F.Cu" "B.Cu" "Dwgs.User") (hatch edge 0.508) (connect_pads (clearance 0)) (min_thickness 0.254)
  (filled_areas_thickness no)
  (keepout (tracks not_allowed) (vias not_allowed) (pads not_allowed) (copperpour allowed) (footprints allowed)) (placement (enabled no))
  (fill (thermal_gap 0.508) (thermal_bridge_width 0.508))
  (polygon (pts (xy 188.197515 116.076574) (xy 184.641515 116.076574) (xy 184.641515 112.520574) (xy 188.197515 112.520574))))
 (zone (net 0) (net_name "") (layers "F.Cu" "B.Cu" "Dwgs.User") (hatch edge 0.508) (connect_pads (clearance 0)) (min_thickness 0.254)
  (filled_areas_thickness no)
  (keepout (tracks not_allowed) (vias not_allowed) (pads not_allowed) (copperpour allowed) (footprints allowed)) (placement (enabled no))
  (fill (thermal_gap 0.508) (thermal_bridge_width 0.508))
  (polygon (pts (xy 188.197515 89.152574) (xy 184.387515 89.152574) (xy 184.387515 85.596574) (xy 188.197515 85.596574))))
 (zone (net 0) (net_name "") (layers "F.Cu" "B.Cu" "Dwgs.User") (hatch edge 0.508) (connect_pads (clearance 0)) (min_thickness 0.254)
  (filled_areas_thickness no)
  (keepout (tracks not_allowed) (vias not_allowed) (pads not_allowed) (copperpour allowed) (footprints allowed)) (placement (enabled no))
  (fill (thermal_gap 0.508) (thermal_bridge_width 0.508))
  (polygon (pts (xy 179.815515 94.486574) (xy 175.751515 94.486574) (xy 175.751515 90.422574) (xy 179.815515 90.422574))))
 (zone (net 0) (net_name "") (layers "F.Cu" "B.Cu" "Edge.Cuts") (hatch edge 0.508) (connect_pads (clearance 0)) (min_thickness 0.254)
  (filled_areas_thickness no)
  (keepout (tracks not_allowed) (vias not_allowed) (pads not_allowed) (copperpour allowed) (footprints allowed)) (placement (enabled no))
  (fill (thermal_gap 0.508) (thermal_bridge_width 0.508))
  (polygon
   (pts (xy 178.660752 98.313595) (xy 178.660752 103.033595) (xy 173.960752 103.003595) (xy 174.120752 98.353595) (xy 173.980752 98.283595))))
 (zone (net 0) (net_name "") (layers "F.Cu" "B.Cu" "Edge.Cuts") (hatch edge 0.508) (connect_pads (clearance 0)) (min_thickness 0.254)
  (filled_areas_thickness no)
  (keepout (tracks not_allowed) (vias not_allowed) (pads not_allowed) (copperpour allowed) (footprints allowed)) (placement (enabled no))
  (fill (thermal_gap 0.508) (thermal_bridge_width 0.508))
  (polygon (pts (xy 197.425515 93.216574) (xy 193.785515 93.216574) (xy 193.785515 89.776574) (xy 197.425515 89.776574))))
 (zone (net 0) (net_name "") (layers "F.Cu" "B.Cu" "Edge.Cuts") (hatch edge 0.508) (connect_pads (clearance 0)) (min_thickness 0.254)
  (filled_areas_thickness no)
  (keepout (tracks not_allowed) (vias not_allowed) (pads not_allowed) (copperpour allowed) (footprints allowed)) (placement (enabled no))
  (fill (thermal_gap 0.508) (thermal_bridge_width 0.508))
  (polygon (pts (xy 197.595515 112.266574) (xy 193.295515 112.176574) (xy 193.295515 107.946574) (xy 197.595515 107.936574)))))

